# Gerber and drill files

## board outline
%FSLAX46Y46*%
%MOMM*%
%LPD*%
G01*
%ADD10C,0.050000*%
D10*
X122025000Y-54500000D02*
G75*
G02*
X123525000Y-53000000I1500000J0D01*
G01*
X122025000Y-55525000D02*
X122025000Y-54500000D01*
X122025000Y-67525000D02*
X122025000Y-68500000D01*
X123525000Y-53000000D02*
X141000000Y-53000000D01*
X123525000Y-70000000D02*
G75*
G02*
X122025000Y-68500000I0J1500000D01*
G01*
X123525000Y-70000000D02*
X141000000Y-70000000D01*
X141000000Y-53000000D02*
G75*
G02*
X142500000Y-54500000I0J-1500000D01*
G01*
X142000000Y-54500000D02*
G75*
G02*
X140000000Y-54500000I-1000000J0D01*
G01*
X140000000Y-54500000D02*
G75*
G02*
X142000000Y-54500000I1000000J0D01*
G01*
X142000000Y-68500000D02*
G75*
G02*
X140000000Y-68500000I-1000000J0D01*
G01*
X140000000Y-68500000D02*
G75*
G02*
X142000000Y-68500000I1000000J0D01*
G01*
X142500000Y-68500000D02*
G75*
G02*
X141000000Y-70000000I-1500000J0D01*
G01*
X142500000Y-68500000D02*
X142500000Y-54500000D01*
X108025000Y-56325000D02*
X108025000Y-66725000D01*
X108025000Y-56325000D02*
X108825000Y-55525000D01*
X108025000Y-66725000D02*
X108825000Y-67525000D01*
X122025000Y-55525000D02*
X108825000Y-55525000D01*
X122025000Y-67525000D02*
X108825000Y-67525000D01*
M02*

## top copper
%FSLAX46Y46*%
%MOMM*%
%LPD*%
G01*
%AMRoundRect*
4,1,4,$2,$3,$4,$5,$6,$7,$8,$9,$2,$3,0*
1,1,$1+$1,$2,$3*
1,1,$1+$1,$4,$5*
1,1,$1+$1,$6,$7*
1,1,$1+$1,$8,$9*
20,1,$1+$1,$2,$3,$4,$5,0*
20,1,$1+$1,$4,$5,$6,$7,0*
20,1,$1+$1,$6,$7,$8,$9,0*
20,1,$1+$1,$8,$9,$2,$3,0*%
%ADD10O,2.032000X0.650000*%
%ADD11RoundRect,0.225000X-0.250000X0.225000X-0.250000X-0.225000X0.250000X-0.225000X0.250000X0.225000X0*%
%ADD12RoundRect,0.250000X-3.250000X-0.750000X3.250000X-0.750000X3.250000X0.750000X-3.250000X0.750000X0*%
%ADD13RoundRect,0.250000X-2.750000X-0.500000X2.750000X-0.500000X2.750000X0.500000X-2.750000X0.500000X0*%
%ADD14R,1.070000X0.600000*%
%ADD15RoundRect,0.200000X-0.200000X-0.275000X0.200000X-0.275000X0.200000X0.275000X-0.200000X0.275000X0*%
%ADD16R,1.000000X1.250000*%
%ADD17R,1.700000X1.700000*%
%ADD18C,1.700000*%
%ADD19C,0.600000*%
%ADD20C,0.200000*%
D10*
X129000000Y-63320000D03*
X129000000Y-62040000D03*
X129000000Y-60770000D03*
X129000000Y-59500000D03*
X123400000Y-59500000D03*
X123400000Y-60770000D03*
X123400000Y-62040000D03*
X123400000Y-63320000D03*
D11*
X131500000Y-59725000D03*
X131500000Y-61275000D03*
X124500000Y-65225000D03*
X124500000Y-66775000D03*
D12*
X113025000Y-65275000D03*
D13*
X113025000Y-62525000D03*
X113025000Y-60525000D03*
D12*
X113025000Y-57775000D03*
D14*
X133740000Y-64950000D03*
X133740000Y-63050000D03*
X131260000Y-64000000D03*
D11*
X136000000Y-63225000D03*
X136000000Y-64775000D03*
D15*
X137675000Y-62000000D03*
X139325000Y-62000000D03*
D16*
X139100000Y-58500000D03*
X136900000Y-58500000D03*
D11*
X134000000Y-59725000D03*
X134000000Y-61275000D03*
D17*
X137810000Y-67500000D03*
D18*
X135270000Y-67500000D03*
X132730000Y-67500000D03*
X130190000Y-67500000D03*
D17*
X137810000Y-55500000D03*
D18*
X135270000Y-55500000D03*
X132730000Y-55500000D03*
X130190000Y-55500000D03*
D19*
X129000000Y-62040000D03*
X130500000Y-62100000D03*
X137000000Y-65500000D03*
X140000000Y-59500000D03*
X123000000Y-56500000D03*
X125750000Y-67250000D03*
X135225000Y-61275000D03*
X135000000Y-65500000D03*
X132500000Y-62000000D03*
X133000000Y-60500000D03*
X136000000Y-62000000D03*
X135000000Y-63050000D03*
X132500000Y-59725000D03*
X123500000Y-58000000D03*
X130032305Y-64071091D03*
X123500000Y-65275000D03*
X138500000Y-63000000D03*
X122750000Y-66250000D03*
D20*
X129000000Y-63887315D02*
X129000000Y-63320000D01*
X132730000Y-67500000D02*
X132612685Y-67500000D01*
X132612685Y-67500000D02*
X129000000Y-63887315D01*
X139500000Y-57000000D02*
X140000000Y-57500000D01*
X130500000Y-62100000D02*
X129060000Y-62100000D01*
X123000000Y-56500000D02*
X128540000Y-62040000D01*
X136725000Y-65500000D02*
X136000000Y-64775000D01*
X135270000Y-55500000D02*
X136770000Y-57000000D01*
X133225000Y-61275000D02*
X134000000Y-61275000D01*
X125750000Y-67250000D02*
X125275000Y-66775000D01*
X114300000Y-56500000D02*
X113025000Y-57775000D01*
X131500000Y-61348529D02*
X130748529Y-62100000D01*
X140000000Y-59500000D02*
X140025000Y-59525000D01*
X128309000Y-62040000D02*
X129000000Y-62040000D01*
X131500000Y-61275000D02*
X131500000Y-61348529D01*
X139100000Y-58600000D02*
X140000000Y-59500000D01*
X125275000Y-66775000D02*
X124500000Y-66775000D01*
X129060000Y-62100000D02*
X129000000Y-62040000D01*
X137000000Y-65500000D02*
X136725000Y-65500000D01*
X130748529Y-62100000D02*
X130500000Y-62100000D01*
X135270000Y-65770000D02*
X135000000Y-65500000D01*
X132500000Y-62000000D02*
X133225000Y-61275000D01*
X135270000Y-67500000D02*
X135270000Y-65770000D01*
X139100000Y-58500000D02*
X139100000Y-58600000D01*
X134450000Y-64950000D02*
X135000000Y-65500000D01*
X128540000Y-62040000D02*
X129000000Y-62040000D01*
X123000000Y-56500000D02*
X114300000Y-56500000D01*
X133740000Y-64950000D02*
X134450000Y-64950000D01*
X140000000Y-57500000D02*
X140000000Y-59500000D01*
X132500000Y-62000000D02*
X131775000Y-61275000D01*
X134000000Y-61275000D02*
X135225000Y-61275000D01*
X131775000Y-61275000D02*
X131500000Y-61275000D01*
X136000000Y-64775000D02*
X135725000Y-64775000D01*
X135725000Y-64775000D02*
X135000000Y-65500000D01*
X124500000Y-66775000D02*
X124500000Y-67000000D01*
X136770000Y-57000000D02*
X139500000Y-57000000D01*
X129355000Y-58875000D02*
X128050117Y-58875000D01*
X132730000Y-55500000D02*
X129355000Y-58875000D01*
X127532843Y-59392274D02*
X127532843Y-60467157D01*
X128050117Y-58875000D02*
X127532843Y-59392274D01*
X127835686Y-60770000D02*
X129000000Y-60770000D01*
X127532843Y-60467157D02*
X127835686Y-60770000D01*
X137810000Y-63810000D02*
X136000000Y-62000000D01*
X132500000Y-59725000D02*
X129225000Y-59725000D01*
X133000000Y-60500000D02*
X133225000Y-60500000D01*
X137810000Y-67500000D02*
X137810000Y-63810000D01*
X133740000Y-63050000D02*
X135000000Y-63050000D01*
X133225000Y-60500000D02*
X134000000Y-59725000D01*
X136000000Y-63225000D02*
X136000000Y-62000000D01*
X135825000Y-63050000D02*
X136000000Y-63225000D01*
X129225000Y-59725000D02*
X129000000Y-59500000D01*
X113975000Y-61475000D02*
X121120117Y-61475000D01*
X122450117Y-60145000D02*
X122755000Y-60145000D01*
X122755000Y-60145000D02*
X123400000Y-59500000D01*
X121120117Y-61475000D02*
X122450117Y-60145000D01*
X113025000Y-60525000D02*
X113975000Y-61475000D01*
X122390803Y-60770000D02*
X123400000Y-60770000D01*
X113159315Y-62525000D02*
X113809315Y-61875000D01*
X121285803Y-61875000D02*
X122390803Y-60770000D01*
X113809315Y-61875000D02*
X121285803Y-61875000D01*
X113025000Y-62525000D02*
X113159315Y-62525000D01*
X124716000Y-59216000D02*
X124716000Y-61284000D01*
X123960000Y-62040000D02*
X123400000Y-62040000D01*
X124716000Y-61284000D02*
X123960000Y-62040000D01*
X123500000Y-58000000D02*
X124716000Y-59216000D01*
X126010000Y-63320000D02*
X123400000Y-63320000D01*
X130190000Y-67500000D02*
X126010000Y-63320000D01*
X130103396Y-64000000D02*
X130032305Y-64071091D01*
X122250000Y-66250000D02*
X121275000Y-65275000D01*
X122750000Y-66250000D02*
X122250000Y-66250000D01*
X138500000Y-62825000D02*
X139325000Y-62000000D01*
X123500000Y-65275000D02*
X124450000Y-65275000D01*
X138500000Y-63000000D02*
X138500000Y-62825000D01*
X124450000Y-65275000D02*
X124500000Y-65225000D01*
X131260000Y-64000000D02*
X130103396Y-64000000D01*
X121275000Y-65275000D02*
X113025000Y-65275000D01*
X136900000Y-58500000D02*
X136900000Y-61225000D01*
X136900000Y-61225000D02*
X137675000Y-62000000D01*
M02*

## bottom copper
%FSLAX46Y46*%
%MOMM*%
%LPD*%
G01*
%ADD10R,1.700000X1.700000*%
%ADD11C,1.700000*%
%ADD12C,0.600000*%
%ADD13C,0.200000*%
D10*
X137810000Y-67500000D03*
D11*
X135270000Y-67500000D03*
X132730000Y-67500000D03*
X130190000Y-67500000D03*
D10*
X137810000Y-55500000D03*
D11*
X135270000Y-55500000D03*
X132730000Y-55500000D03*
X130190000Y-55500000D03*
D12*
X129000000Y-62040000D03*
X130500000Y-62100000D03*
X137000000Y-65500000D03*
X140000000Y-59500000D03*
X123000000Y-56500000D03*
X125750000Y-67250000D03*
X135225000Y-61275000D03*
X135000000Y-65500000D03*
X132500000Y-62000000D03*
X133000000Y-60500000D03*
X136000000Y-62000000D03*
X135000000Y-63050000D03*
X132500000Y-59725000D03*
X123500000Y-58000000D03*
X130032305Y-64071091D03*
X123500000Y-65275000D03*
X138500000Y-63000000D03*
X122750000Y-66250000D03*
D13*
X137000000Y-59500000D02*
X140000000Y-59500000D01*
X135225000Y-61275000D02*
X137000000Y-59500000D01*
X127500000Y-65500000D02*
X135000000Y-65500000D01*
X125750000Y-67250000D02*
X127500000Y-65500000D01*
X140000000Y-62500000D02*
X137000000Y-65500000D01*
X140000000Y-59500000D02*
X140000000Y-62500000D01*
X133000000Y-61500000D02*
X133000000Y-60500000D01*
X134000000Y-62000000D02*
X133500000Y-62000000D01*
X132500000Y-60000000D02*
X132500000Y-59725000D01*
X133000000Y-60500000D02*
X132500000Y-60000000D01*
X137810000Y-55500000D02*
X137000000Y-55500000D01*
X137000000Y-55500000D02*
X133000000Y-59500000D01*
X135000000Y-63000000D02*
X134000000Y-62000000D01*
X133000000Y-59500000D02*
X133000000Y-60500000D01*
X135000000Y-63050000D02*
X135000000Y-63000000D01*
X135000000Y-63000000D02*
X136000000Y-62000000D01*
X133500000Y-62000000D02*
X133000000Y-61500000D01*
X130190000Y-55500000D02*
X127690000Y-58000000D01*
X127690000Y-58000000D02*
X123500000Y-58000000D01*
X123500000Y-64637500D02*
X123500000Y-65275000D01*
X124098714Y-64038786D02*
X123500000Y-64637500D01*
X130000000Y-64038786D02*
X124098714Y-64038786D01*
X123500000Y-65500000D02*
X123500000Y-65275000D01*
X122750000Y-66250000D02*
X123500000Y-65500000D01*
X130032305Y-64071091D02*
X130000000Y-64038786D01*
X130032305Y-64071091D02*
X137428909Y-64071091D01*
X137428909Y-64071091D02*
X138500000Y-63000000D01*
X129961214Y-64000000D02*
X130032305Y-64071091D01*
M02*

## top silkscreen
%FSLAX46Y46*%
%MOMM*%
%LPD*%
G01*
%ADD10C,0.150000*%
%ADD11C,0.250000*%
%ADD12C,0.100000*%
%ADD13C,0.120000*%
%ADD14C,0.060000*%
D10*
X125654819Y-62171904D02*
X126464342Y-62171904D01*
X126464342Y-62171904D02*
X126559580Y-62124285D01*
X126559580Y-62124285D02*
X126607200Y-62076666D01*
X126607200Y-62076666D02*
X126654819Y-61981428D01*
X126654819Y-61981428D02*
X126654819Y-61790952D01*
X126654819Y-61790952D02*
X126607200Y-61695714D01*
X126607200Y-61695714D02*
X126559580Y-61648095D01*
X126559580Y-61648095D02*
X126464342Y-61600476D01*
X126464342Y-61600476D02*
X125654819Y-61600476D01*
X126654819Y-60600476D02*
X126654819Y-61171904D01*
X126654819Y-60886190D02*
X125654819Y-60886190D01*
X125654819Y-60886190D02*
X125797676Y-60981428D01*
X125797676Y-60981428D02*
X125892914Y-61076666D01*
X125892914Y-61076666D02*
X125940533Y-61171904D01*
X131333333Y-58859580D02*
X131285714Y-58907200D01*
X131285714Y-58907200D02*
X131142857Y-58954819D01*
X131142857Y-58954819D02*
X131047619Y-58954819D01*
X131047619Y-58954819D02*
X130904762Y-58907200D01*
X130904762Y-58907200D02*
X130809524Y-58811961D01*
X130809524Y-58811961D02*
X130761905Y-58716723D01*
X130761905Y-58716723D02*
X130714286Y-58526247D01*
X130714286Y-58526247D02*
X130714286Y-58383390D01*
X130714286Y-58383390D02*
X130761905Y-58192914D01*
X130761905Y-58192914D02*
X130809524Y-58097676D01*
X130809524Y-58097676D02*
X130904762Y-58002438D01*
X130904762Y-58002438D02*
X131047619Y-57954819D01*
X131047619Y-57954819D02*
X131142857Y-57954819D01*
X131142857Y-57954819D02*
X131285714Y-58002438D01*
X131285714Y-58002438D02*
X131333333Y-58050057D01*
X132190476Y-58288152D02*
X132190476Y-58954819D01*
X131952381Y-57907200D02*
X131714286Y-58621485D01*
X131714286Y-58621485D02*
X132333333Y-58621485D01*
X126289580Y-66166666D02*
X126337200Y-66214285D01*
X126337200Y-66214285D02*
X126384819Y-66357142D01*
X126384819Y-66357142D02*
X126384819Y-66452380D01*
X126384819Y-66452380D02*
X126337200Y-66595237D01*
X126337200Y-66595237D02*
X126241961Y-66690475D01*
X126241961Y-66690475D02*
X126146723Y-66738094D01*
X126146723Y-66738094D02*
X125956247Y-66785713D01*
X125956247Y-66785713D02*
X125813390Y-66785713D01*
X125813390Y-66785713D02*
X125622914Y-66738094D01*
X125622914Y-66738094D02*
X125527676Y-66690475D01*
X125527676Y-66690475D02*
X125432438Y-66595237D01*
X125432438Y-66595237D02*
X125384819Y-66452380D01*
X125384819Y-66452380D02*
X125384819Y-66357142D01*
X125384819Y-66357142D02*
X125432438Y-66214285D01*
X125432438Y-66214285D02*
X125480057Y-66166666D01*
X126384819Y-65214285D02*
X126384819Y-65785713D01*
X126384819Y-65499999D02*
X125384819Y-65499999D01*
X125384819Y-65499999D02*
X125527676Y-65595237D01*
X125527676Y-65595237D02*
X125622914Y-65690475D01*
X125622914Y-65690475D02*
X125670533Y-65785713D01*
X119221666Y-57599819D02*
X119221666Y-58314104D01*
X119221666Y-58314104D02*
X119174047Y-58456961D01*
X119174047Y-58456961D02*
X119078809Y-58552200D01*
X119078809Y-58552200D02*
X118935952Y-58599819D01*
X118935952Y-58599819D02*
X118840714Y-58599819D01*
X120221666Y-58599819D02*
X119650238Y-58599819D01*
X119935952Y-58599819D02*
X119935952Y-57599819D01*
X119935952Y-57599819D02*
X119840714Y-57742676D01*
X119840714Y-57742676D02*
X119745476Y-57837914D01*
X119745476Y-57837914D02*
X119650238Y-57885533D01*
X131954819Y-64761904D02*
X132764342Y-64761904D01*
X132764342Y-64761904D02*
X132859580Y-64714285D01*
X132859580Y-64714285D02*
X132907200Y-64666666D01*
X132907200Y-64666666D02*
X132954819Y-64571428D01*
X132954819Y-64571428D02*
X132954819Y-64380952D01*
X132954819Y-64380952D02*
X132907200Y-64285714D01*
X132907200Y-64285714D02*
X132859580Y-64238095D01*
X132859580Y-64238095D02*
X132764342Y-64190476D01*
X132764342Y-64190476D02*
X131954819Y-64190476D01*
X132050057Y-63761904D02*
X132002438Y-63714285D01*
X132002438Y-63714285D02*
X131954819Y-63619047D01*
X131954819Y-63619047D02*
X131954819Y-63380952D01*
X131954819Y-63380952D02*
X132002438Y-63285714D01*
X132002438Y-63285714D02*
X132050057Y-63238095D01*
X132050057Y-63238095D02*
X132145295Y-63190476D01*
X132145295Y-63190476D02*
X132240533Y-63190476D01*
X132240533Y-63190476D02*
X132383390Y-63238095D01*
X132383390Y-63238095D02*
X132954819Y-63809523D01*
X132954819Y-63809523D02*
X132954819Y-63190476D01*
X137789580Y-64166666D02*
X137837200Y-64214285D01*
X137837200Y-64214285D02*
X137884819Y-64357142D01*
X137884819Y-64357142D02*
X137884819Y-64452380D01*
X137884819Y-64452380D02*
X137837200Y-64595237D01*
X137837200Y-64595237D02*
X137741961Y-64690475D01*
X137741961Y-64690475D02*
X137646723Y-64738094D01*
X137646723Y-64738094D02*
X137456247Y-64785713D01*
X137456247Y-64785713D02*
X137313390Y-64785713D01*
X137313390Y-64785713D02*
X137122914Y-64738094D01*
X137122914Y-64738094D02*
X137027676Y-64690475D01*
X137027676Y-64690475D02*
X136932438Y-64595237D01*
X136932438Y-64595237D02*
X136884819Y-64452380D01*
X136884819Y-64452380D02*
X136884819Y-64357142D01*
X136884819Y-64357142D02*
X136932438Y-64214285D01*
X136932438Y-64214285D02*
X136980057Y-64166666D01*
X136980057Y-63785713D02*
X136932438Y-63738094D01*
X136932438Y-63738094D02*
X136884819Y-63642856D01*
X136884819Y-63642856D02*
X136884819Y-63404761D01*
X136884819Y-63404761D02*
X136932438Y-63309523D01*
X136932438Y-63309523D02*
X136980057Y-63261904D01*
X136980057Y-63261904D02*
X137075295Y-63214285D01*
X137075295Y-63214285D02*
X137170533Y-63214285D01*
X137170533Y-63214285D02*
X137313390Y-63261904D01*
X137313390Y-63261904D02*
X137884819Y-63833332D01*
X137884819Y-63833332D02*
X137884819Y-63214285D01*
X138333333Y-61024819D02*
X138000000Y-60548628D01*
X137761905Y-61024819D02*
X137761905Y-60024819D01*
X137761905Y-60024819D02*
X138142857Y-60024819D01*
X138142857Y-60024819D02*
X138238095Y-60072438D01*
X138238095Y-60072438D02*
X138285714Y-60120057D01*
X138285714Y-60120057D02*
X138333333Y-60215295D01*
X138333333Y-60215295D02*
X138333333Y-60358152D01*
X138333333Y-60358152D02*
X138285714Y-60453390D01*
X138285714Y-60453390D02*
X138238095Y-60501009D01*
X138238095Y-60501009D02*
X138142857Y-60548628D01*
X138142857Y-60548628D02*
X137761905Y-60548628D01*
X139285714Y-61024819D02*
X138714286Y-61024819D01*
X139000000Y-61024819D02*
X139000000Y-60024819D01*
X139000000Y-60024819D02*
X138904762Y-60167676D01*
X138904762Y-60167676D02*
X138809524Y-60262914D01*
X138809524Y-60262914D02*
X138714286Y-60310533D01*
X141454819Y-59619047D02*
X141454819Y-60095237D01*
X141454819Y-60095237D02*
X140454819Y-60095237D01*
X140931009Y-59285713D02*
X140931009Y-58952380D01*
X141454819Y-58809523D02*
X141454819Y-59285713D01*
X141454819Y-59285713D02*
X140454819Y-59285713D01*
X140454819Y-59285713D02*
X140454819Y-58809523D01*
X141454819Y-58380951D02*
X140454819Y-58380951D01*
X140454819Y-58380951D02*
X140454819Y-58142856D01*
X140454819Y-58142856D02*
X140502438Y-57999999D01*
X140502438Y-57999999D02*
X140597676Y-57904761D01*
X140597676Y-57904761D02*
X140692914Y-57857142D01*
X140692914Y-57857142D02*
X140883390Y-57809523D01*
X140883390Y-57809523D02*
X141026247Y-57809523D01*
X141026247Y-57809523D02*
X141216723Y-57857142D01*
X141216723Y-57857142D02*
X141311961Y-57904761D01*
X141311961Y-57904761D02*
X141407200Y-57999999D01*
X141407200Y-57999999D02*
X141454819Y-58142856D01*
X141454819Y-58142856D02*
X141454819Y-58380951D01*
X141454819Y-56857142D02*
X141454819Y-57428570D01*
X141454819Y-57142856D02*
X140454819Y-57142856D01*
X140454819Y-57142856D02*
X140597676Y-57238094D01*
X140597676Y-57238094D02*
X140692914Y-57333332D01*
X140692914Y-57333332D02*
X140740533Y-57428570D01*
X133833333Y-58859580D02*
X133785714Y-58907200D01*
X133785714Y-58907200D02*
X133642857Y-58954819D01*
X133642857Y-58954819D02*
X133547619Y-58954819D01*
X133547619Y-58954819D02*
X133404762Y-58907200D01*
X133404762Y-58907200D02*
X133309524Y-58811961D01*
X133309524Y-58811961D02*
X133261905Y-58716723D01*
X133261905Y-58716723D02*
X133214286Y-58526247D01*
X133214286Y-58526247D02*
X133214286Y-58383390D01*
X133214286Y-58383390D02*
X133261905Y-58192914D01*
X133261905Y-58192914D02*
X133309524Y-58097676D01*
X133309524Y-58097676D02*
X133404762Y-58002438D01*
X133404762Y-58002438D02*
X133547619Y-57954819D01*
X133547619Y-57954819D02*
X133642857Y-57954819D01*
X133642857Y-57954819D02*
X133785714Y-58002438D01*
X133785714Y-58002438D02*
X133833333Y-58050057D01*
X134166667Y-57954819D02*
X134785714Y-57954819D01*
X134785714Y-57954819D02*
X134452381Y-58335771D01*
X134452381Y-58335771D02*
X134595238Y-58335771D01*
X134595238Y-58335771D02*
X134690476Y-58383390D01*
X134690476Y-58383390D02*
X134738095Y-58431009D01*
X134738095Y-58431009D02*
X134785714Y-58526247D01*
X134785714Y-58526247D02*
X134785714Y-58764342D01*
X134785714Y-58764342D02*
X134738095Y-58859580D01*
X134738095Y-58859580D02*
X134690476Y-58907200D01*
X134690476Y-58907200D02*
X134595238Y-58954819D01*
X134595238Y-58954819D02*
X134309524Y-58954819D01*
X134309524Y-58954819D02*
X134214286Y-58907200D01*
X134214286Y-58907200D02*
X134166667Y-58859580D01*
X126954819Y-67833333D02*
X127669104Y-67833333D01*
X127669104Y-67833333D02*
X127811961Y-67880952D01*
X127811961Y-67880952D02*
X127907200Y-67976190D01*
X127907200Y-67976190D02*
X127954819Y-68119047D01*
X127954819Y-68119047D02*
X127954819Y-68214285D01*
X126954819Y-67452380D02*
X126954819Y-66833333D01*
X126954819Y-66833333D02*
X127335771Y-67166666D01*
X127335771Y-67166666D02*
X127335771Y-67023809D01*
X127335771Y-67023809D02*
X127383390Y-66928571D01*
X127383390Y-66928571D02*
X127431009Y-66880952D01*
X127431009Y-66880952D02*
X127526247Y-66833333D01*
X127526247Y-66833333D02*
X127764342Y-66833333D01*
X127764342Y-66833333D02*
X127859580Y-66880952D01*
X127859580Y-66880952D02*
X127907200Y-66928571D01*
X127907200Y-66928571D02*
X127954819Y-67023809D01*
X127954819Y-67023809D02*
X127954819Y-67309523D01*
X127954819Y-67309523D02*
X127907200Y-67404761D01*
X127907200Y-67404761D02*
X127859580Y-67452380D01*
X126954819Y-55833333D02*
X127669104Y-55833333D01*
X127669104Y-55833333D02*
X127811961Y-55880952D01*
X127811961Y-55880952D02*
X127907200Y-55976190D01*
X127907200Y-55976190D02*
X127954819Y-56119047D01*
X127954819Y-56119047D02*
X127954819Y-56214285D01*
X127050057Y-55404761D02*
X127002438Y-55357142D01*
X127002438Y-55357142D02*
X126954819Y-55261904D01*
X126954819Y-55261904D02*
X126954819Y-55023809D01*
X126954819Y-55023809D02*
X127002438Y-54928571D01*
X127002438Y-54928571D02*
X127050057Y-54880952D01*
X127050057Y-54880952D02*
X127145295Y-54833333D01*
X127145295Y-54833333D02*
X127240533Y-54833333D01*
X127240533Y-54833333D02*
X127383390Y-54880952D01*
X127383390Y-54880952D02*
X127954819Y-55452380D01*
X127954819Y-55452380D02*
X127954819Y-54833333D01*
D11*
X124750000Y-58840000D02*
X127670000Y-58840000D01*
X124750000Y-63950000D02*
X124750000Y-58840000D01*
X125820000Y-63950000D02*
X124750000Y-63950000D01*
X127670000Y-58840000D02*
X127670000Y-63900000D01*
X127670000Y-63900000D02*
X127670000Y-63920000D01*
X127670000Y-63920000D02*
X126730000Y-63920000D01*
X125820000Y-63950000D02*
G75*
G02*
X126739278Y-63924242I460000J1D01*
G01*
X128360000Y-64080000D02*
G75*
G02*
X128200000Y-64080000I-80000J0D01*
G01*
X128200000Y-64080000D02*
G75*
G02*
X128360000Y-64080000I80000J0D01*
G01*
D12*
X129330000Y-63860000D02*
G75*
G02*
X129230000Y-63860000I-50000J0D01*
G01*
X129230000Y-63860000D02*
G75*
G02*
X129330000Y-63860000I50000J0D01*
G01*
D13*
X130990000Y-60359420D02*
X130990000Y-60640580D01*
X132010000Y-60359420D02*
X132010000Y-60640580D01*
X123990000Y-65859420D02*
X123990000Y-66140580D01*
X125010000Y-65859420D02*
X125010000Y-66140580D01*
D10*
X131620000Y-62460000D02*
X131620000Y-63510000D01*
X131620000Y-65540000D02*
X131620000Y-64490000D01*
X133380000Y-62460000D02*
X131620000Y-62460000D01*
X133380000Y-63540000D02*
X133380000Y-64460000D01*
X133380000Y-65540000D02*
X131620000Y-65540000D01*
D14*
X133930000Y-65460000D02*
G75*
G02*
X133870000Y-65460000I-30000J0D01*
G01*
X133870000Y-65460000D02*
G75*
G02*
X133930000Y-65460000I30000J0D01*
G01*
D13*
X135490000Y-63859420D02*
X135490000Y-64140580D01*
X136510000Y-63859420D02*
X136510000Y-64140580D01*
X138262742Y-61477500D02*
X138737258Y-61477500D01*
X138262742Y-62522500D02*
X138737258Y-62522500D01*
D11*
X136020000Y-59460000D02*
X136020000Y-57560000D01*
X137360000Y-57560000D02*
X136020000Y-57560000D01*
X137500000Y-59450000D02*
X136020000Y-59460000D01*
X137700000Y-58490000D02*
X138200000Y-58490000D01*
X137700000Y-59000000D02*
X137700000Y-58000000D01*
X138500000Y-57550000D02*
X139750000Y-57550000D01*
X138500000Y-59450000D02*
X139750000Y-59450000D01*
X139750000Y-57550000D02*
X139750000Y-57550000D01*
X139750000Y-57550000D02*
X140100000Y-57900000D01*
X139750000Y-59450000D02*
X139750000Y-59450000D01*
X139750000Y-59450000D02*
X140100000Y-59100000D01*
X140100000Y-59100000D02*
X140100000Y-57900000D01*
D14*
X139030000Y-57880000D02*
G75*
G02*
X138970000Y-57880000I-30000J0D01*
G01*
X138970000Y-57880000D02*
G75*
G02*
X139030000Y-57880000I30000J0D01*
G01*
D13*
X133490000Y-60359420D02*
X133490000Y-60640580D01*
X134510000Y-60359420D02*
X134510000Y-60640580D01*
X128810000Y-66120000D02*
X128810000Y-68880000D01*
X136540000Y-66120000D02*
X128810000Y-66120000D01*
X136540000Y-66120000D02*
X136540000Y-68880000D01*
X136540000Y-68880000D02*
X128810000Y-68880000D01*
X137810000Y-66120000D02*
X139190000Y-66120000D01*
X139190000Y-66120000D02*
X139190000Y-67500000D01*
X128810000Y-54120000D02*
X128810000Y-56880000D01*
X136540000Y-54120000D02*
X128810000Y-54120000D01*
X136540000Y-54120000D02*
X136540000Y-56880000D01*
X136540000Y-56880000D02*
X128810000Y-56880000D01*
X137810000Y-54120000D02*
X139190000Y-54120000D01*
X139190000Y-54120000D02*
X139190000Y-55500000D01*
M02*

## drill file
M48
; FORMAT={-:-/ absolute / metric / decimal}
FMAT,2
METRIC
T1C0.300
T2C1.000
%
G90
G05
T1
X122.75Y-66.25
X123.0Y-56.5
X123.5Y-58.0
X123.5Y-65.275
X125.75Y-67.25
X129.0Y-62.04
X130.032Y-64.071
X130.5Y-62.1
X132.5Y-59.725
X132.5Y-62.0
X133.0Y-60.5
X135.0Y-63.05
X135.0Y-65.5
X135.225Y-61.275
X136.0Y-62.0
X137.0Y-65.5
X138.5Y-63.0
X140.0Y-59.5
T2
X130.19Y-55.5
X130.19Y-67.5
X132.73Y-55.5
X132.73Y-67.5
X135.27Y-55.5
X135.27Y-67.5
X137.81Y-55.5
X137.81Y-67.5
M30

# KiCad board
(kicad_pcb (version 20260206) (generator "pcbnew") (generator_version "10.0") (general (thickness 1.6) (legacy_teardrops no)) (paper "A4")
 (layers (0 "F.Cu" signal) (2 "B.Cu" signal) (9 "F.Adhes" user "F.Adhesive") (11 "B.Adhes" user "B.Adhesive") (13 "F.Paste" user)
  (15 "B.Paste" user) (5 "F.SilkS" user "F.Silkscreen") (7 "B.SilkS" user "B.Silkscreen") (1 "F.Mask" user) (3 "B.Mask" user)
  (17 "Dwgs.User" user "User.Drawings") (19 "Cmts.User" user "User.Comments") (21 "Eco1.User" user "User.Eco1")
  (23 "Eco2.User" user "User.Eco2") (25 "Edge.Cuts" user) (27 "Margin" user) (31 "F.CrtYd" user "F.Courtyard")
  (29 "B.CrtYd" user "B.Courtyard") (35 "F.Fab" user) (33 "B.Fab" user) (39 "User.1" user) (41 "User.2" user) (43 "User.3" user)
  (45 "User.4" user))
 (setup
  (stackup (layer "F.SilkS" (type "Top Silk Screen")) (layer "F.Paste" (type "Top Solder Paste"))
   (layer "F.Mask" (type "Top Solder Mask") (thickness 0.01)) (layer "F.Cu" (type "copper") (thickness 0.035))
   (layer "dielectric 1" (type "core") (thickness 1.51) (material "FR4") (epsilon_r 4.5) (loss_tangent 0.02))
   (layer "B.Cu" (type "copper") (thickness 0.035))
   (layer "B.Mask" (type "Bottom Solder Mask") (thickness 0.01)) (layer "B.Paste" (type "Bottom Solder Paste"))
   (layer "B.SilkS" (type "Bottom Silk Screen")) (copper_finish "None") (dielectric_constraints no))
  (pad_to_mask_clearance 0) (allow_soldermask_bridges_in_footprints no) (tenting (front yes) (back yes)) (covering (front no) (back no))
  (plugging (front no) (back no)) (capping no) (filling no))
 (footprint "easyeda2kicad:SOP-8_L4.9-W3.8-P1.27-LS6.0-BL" (layer "F.Cu") (at 126.2 61.41 90)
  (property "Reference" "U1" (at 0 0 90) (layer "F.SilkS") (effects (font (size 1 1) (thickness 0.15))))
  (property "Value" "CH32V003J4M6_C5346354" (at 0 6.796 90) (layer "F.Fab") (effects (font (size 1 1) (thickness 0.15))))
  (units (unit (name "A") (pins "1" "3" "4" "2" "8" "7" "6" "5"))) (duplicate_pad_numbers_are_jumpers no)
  (fp_line (start 2.57 -1.45) (end 2.57 1.47) (stroke (width 0.25) (type solid)) (layer "F.SilkS"))
  (fp_line (start -2.54 -1.45) (end 2.57 -1.45) (stroke (width 0.25) (type solid)) (layer "F.SilkS"))
  (fp_line (start -2.54 -0.38) (end -2.54 -1.45) (stroke (width 0.25) (type solid)) (layer "F.SilkS"))
  (fp_line (start 2.57 1.47) (end -2.49 1.47) (stroke (width 0.25) (type solid)) (layer "F.SilkS"))
  (fp_line (start -2.49 1.47) (end -2.51 1.47) (stroke (width 0.25) (type solid)) (layer "F.SilkS"))
  (fp_line (start -2.51 1.47) (end -2.51 0.53) (stroke (width 0.25) (type solid)) (layer "F.SilkS"))
  (fp_arc (start -2.54 -0.38) (mid -2.08018 0.067116) (end -2.514242 0.539278) (stroke (width 0.25) (type solid)) (layer "F.SilkS"))
  (fp_circle (center -2.67 2.08) (end -2.59 2.08) (stroke (width 0.25) (type solid)) (fill no) (layer "F.SilkS"))
  (fp_circle (center -2.45 3.08) (end -2.4 3.08) (stroke (width 0.1) (type solid)) (fill no) (layer "F.SilkS"))
  (pad "1" smd oval (at -1.91 2.8 90) (size 0.65 2.032) (layers "F.Cu" "F.Mask" "F.Paste") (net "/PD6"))
  (pad "2" smd oval (at -0.63 2.8 90) (size 0.65 2.032) (layers "F.Cu" "F.Mask" "F.Paste") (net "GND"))
  (pad "3" smd oval (at 0.64 2.8 90) (size 0.65 2.032) (layers "F.Cu" "F.Mask" "F.Paste") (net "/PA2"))
  (pad "4" smd oval (at 1.91 2.8 90) (size 0.65 2.032) (layers "F.Cu" "F.Mask" "F.Paste") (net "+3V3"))
  (pad "5" smd oval (at 1.91 -2.8 90) (size 0.65 2.032) (layers "F.Cu" "F.Mask" "F.Paste") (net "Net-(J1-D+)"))
  (pad "6" smd oval (at 0.64 -2.8 90) (size 0.65 2.032) (layers "F.Cu" "F.Mask" "F.Paste") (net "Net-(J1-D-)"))
  (pad "7" smd oval (at -0.63 -2.8 90) (size 0.65 2.032) (layers "F.Cu" "F.Mask" "F.Paste") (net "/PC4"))
  (pad "8" smd oval (at -1.91 -2.8 90) (size 0.65 2.032) (layers "F.Cu" "F.Mask" "F.Paste") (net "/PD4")))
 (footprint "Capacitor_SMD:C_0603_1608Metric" (layer "F.Cu") (at 131.5 60.5 -90)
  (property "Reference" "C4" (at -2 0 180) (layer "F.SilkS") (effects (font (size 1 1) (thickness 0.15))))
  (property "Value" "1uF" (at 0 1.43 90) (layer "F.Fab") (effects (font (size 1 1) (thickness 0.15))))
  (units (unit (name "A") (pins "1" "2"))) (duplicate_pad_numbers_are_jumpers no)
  (fp_line (start -0.14058 0.51) (end 0.14058 0.51) (stroke (width 0.12) (type solid)) (layer "F.SilkS"))
  (fp_line (start -0.14058 -0.51) (end 0.14058 -0.51) (stroke (width 0.12) (type solid)) (layer "F.SilkS"))
  (pad "1" smd roundrect (at -0.775 0 270) (size 0.9 0.95) (layers "F.Cu" "F.Mask" "F.Paste") (roundrect_rratio 0.25) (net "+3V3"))
  (pad "2" smd roundrect (at 0.775 0 270) (size 0.9 0.95) (layers "F.Cu" "F.Mask" "F.Paste") (roundrect_rratio 0.25) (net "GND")))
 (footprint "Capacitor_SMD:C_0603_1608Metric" (layer "F.Cu") (at 124.5 66 -90)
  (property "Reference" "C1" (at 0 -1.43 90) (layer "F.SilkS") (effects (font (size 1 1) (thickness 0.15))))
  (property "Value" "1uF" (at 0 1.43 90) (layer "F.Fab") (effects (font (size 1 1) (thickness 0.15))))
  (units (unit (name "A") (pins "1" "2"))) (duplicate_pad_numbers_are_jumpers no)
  (fp_line (start -0.14058 0.51) (end 0.14058 0.51) (stroke (width 0.12) (type solid)) (layer "F.SilkS"))
  (fp_line (start -0.14058 -0.51) (end 0.14058 -0.51) (stroke (width 0.12) (type solid)) (layer "F.SilkS"))
  (pad "1" smd roundrect (at -0.775 0 270) (size 0.9 0.95) (layers "F.Cu" "F.Mask" "F.Paste") (roundrect_rratio 0.25) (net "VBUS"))
  (pad "2" smd roundrect (at 0.775 0 270) (size 0.9 0.95) (layers "F.Cu" "F.Mask" "F.Paste") (roundrect_rratio 0.25) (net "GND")))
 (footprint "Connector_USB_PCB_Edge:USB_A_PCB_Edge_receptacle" (layer "F.Cu") (at 113.025 61.525)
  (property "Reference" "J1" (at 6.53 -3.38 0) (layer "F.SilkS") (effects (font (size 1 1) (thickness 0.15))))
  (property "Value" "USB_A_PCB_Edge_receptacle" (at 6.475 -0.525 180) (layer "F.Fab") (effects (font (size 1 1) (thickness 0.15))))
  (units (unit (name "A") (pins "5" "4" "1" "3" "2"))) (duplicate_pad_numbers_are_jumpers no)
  (fp_line (start -5 -5.2) (end -5 5.2) (stroke (width 0.05) (type default)) (layer "Edge.Cuts"))
  (fp_line (start -5 -5.2) (end -4.2 -6) (stroke (width 0.05) (type default)) (layer "Edge.Cuts"))
  (fp_line (start -5 5.2) (end -4.2 6) (stroke (width 0.05) (type default)) (layer "Edge.Cuts"))
  (fp_line (start 9 -6) (end -4.2 -6) (stroke (width 0.05) (type default)) (layer "Edge.Cuts"))
  (fp_line (start 9 6) (end -4.2 6) (stroke (width 0.05) (type default)) (layer "Edge.Cuts"))
  (pad "1" smd roundrect (at 0 3.75) (size 7 2) (layers "F.Cu" "F.Mask") (roundrect_rratio 0.125) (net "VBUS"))
  (pad "2" smd roundrect (at 0 1) (size 6 1.5) (layers "F.Cu" "F.Mask") (roundrect_rratio 0.1666666667) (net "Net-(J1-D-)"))
  (pad "3" smd roundrect (at 0 -1) (size 6 1.5) (layers "F.Cu" "F.Mask") (roundrect_rratio 0.1666666667) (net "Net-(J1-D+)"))
  (pad "4" smd roundrect (at 0 -3.75) (size 7 2) (layers "F.Cu" "F.Mask") (roundrect_rratio 0.125) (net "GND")))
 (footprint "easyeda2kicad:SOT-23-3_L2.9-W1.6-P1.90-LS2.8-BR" (layer "F.Cu") (at 132.5 64)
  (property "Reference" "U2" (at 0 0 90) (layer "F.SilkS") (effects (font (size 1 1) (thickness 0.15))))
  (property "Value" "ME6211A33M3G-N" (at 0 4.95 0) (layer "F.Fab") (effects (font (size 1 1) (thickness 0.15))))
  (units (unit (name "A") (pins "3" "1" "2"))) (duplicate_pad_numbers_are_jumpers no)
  (fp_line (start -0.88 -1.54) (end -0.88 -0.49) (stroke (width 0.15) (type solid)) (layer "F.SilkS"))
  (fp_line (start -0.88 1.54) (end -0.88 0.49) (stroke (width 0.15) (type solid)) (layer "F.SilkS"))
  (fp_line (start 0.88 -1.54) (end -0.88 -1.54) (stroke (width 0.15) (type solid)) (layer "F.SilkS"))
  (fp_line (start 0.88 -0.46) (end 0.88 0.46) (stroke (width 0.15) (type solid)) (layer "F.SilkS"))
  (fp_line (start 0.88 1.54) (end -0.88 1.54) (stroke (width 0.15) (type solid)) (layer "F.SilkS"))
  (fp_circle (center 1.4 1.46) (end 1.43 1.46) (stroke (width 0.06) (type solid)) (fill no) (layer "F.SilkS"))
  (pad "1" smd rect (at 1.24 0.95) (size 1.07 0.6) (layers "F.Cu" "F.Mask" "F.Paste") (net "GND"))
  (pad "2" smd rect (at 1.24 -0.95) (size 1.07 0.6) (layers "F.Cu" "F.Mask" "F.Paste") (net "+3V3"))
  (pad "3" smd rect (at -1.24 0) (size 1.07 0.6) (layers "F.Cu" "F.Mask" "F.Paste") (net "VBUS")))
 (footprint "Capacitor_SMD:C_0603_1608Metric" (layer "F.Cu") (at 136 64 -90)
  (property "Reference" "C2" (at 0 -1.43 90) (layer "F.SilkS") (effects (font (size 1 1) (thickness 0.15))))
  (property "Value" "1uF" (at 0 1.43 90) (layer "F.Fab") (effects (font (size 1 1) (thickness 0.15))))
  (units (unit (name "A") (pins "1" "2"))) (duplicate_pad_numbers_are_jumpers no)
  (fp_line (start -0.14058 0.51) (end 0.14058 0.51) (stroke (width 0.12) (type solid)) (layer "F.SilkS"))
  (fp_line (start -0.14058 -0.51) (end 0.14058 -0.51) (stroke (width 0.12) (type solid)) (layer "F.SilkS"))
  (pad "1" smd roundrect (at -0.775 0 270) (size 0.9 0.95) (layers "F.Cu" "F.Mask" "F.Paste") (roundrect_rratio 0.25) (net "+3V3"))
  (pad "2" smd roundrect (at 0.775 0 270) (size 0.9 0.95) (layers "F.Cu" "F.Mask" "F.Paste") (roundrect_rratio 0.25) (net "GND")))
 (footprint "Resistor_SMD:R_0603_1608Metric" (layer "F.Cu") (at 138.5 62)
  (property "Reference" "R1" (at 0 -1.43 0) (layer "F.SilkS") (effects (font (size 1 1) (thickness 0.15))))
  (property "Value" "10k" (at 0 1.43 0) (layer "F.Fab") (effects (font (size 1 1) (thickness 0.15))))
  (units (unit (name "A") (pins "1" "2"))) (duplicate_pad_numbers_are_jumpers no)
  (fp_line (start -0.237258 -0.5225) (end 0.237258 -0.5225) (stroke (width 0.12) (type solid)) (layer "F.SilkS"))
  (fp_line (start -0.237258 0.5225) (end 0.237258 0.5225) (stroke (width 0.12) (type solid)) (layer "F.SilkS"))
  (pad "1" smd roundrect (at -0.825 0) (size 0.8 0.95) (layers "F.Cu" "F.Mask" "F.Paste") (roundrect_rratio 0.25) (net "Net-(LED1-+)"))
  (pad "2" smd roundrect (at 0.825 0) (size 0.8 0.95) (layers "F.Cu" "F.Mask" "F.Paste") (roundrect_rratio 0.25) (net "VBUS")))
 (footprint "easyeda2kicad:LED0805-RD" (layer "F.Cu") (at 138 58.5 180)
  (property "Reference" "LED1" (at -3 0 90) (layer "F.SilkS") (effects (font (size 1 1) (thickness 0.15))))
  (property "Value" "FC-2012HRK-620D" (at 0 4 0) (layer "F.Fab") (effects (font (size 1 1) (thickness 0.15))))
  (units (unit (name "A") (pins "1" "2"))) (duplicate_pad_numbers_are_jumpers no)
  (fp_line (start 1.98 -0.96) (end 1.98 0.94) (stroke (width 0.25) (type solid)) (layer "F.SilkS"))
  (fp_line (start 0.64 0.94) (end 1.98 0.94) (stroke (width 0.25) (type solid)) (layer "F.SilkS"))
  (fp_line (start 0.5 -0.95) (end 1.98 -0.96) (stroke (width 0.25) (type solid)) (layer "F.SilkS"))
  (fp_line (start 0.3 0.01) (end -0.2 0.01) (stroke (width 0.25) (type solid)) (layer "F.SilkS"))
  (fp_line (start 0.3 -0.5) (end 0.3 0.5) (stroke (width 0.25) (type solid)) (layer "F.SilkS"))
  (fp_line (start -0.5 0.95) (end -1.75 0.95) (stroke (width 0.25) (type solid)) (layer "F.SilkS"))
  (fp_line (start -0.5 -0.95) (end -1.75 -0.95) (stroke (width 0.25) (type solid)) (layer "F.SilkS"))
  (fp_line (start -1.75 0.95) (end -1.75 0.95) (stroke (width 0.25) (type solid)) (layer "F.SilkS"))
  (fp_line (start -1.75 0.95) (end -2.1 0.6) (stroke (width 0.25) (type solid)) (layer "F.SilkS"))
  (fp_line (start -1.75 -0.95) (end -1.75 -0.95) (stroke (width 0.25) (type solid)) (layer "F.SilkS"))
  (fp_line (start -1.75 -0.95) (end -2.1 -0.6) (stroke (width 0.25) (type solid)) (layer "F.SilkS"))
  (fp_line (start -2.1 -0.6) (end -2.1 0.6) (stroke (width 0.25) (type solid)) (layer "F.SilkS"))
  (fp_circle (center -1 0.62) (end -0.97 0.62) (stroke (width 0.06) (type solid)) (fill no) (layer "F.SilkS"))
  (pad "1" smd rect (at -1.1 0) (size 1 1.25) (layers "F.Cu" "F.Mask" "F.Paste") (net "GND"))
  (pad "2" smd rect (at 1.1 0) (size 1 1.25) (layers "F.Cu" "F.Mask" "F.Paste") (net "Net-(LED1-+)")))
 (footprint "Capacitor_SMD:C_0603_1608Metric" (layer "F.Cu") (at 134 60.5 -90)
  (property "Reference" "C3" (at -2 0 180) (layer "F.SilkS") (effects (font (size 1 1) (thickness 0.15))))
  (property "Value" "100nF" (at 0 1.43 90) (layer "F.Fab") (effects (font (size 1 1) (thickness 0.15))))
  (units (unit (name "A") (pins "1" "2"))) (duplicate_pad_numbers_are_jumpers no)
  (fp_line (start -0.14058 0.51) (end 0.14058 0.51) (stroke (width 0.12) (type solid)) (layer "F.SilkS"))
  (fp_line (start -0.14058 -0.51) (end 0.14058 -0.51) (stroke (width 0.12) (type solid)) (layer "F.SilkS"))
  (pad "1" smd roundrect (at -0.775 0 270) (size 0.9 0.95) (layers "F.Cu" "F.Mask" "F.Paste") (roundrect_rratio 0.25) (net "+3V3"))
  (pad "2" smd roundrect (at 0.775 0 270) (size 0.9 0.95) (layers "F.Cu" "F.Mask" "F.Paste") (roundrect_rratio 0.25) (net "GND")))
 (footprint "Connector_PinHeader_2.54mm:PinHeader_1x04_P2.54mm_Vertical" (layer "F.Cu") (at 137.81 67.5 -90)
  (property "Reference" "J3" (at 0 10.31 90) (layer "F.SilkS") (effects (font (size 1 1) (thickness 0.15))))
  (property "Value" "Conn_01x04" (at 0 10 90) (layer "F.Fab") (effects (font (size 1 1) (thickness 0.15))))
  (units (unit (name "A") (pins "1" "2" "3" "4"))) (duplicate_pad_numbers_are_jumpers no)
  (fp_line (start -1.38 9) (end 1.38 9) (stroke (width 0.12) (type solid)) (layer "F.SilkS"))
  (fp_line (start -1.38 1.27) (end -1.38 9) (stroke (width 0.12) (type solid)) (layer "F.SilkS"))
  (fp_line (start -1.38 1.27) (end 1.38 1.27) (stroke (width 0.12) (type solid)) (layer "F.SilkS"))
  (fp_line (start 1.38 1.27) (end 1.38 9) (stroke (width 0.12) (type solid)) (layer "F.SilkS"))
  (fp_line (start -1.38 0) (end -1.38 -1.38) (stroke (width 0.12) (type solid)) (layer "F.SilkS"))
  (fp_line (start -1.38 -1.38) (end 0 -1.38) (stroke (width 0.12) (type solid)) (layer "F.SilkS"))
  (pad "1" thru_hole rect (at 0 0 270) (size 1.7 1.7) (drill 1) (layers "*.Cu" "*.Mask") (remove_unused_layers no) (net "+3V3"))
  (pad "2" thru_hole circle (at 0 2.54 270) (size 1.7 1.7) (drill 1) (layers "*.Cu" "*.Mask") (remove_unused_layers no) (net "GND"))
  (pad "3" thru_hole circle (at 0 5.08 270) (size 1.7 1.7) (drill 1) (layers "*.Cu" "*.Mask") (remove_unused_layers no) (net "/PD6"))
  (pad "4" thru_hole circle (at 0 7.62 270) (size 1.7 1.7) (drill 1) (layers "*.Cu" "*.Mask") (remove_unused_layers no) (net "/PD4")))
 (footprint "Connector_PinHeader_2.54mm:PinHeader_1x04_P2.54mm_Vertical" (layer "F.Cu") (at 137.81 55.5 -90)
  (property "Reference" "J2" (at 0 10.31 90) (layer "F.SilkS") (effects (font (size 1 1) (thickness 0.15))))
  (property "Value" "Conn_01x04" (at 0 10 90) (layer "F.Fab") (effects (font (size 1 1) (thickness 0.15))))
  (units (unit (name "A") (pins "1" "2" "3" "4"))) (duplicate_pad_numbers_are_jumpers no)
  (fp_line (start -1.38 9) (end 1.38 9) (stroke (width 0.12) (type solid)) (layer "F.SilkS"))
  (fp_line (start -1.38 1.27) (end -1.38 9) (stroke (width 0.12) (type solid)) (layer "F.SilkS"))
  (fp_line (start -1.38 1.27) (end 1.38 1.27) (stroke (width 0.12) (type solid)) (layer "F.SilkS"))
  (fp_line (start 1.38 1.27) (end 1.38 9) (stroke (width 0.12) (type solid)) (layer "F.SilkS"))
  (fp_line (start -1.38 0) (end -1.38 -1.38) (stroke (width 0.12) (type solid)) (layer "F.SilkS"))
  (fp_line (start -1.38 -1.38) (end 0 -1.38) (stroke (width 0.12) (type solid)) (layer "F.SilkS"))
  (pad "1" thru_hole rect (at 0 0 270) (size 1.7 1.7) (drill 1) (layers "*.Cu" "*.Mask") (remove_unused_layers no) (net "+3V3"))
  (pad "2" thru_hole circle (at 0 2.54 270) (size 1.7 1.7) (drill 1) (layers "*.Cu" "*.Mask") (remove_unused_layers no) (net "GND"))
  (pad "3" thru_hole circle (at 0 5.08 270) (size 1.7 1.7) (drill 1) (layers "*.Cu" "*.Mask") (remove_unused_layers no) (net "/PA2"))
  (pad "4" thru_hole circle (at 0 7.62 270) (size 1.7 1.7) (drill 1) (layers "*.Cu" "*.Mask") (remove_unused_layers no) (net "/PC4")))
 (gr_arc (start 122.025 54.5) (mid 122.46434 53.43934) (end 123.525 53) (stroke (width 0.05) (type default)) (layer "Edge.Cuts"))
 (gr_line (start 122.025 55.525) (end 122.025 54.5) (stroke (width 0.05) (type default)) (layer "Edge.Cuts"))
 (gr_line (start 122.025 67.525) (end 122.025 68.5) (stroke (width 0.05) (type default)) (layer "Edge.Cuts"))
 (gr_line (start 123.525 53) (end 141 53) (stroke (width 0.05) (type default)) (layer "Edge.Cuts"))
 (gr_arc (start 123.525 70) (mid 122.46434 69.56066) (end 122.025 68.5) (stroke (width 0.05) (type default)) (layer "Edge.Cuts"))
 (gr_line (start 123.525 70) (end 141 70) (stroke (width 0.05) (type default)) (layer "Edge.Cuts"))
 (gr_arc (start 141 53) (mid 142.06066 53.43934) (end 142.5 54.5) (stroke (width 0.05) (type default)) (layer "Edge.Cuts"))
 (gr_circle (center 141 54.5) (end 142 54.5) (stroke (width 0.05) (type solid)) (fill no) (layer "Edge.Cuts"))
 (gr_circle (center 141 68.5) (end 142 68.5) (stroke (width 0.05) (type solid)) (fill no) (layer "Edge.Cuts"))
 (gr_arc (start 142.5 68.5) (mid 142.06066 69.56066) (end 141 70) (stroke (width 0.05) (type default)) (layer "Edge.Cuts"))
 (gr_line (start 142.5 68.5) (end 142.5 54.5) (stroke (width 0.05) (type default)) (layer "Edge.Cuts"))
 (segment (start 129 63.887315) (end 129 63.32) (width 0.2) (layer "F.Cu") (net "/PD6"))
 (segment (start 132.73 67.5) (end 132.612685 67.5) (width 0.2) (layer "F.Cu") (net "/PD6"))
 (segment (start 132.612685 67.5) (end 129 63.887315) (width 0.2) (layer "F.Cu") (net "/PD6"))
 (segment (start 139.5 57) (end 140 57.5) (width 0.2) (layer "F.Cu") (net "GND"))
 (segment (start 130.5 62.1) (end 129.06 62.1) (width 0.2) (layer "F.Cu") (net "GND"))
 (segment (start 123 56.5) (end 128.54 62.04) (width 0.2) (layer "F.Cu") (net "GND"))
 (segment (start 136.725 65.5) (end 136 64.775) (width 0.2) (layer "F.Cu") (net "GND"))
 (segment (start 135.27 55.5) (end 136.77 57) (width 0.2) (layer "F.Cu") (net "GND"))
 (segment (start 133.225 61.275) (end 134 61.275) (width 0.2) (layer "F.Cu") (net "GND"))
 (segment (start 125.75 67.25) (end 125.275 66.775) (width 0.2) (layer "F.Cu") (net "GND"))
 (segment (start 114.3 56.5) (end 113.025 57.775) (width 0.2) (layer "F.Cu") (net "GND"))
 (segment (start 131.5 61.348529) (end 130.748529 62.1) (width 0.2) (layer "F.Cu") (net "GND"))
 (segment (start 140 59.5) (end 140.025 59.525) (width 0.2) (layer "F.Cu") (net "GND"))
 (segment (start 128.309 62.04) (end 129 62.04) (width 0.2) (layer "F.Cu") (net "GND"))
 (segment (start 131.5 61.275) (end 131.5 61.348529) (width 0.2) (layer "F.Cu") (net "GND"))
 (segment (start 139.1 58.6) (end 140 59.5) (width 0.2) (layer "F.Cu") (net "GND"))
 (segment (start 125.275 66.775) (end 124.5 66.775) (width 0.2) (layer "F.Cu") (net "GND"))
 (segment (start 129.06 62.1) (end 129 62.04) (width 0.2) (layer "F.Cu") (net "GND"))
 (segment (start 137 65.5) (end 136.725 65.5) (width 0.2) (layer "F.Cu") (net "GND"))
 (segment (start 130.748529 62.1) (end 130.5 62.1) (width 0.2) (layer "F.Cu") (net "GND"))
 (segment (start 135.27 65.77) (end 135 65.5) (width 0.2) (layer "F.Cu") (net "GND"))
 (segment (start 132.5 62) (end 133.225 61.275) (width 0.2) (layer "F.Cu") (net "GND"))
 (segment (start 135.27 67.5) (end 135.27 65.77) (width 0.2) (layer "F.Cu") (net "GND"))
 (segment (start 139.1 58.5) (end 139.1 58.6) (width 0.2) (layer "F.Cu") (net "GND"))
 (segment (start 134.45 64.95) (end 135 65.5) (width 0.2) (layer "F.Cu") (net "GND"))
 (segment (start 128.54 62.04) (end 129 62.04) (width 0.2) (layer "F.Cu") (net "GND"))
 (segment (start 123 56.5) (end 114.3 56.5) (width 0.2) (layer "F.Cu") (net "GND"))
 (segment (start 133.74 64.95) (end 134.45 64.95) (width 0.2) (layer "F.Cu") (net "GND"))
 (segment (start 140 57.5) (end 140 59.5) (width 0.2) (layer "F.Cu") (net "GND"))
 (segment (start 132.5 62) (end 131.775 61.275) (width 0.2) (layer "F.Cu") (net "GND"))
 (segment (start 134 61.275) (end 135.225 61.275) (width 0.2) (layer "F.Cu") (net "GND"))
 (segment (start 131.775 61.275) (end 131.5 61.275) (width 0.2) (layer "F.Cu") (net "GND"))
 (segment (start 136 64.775) (end 135.725 64.775) (width 0.2) (layer "F.Cu") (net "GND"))
 (segment (start 135.725 64.775) (end 135 65.5) (width 0.2) (layer "F.Cu") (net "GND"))
 (segment (start 124.5 66.775) (end 124.5 67) (width 0.2) (layer "F.Cu") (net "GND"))
 (segment (start 136.77 57) (end 139.5 57) (width 0.2) (layer "F.Cu") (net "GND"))
 (via (at 129 62.04) (size 0.6) (drill 0.3) (layers "F.Cu" "B.Cu") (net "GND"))
 (via (at 130.5 62.1) (size 0.6) (drill 0.3) (layers "F.Cu" "B.Cu") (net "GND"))
 (via (at 137 65.5) (size 0.6) (drill 0.3) (layers "F.Cu" "B.Cu") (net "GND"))
 (via (at 140 59.5) (size 0.6) (drill 0.3) (layers "F.Cu" "B.Cu") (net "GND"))
 (via (at 123 56.5) (size 0.6) (drill 0.3) (layers "F.Cu" "B.Cu") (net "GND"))
 (via (at 125.75 67.25) (size 0.6) (drill 0.3) (layers "F.Cu" "B.Cu") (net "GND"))
 (via (at 135.225 61.275) (size 0.6) (drill 0.3) (layers "F.Cu" "B.Cu") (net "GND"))
 (via (at 135 65.5) (size 0.6) (drill 0.3) (layers "F.Cu" "B.Cu") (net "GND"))
 (via (at 132.5 62) (size 0.6) (drill 0.3) (layers "F.Cu" "B.Cu") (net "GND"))
 (segment (start 137 59.5) (end 140 59.5) (width 0.2) (layer "B.Cu") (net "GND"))
 (segment (start 135.225 61.275) (end 137 59.5) (width 0.2) (layer "B.Cu") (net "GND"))
 (segment (start 127.5 65.5) (end 135 65.5) (width 0.2) (layer "B.Cu") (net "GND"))
 (segment (start 125.75 67.25) (end 127.5 65.5) (width 0.2) (layer "B.Cu") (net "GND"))
 (segment (start 140 62.5) (end 137 65.5) (width 0.2) (layer "B.Cu") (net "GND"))
 (segment (start 140 59.5) (end 140 62.5) (width 0.2) (layer "B.Cu") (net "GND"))
 (segment (start 129.355 58.875) (end 128.050117 58.875) (width 0.2) (layer "F.Cu") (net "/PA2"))
 (segment (start 132.73 55.5) (end 129.355 58.875) (width 0.2) (layer "F.Cu") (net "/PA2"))
 (segment (start 127.532843 59.392274) (end 127.532843 60.467157) (width 0.2) (layer "F.Cu") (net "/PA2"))
 (segment (start 128.050117 58.875) (end 127.532843 59.392274) (width 0.2) (layer "F.Cu") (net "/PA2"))
 (segment (start 127.835686 60.77) (end 129 60.77) (width 0.2) (layer "F.Cu") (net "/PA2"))
 (segment (start 127.532843 60.467157) (end 127.835686 60.77) (width 0.2) (layer "F.Cu") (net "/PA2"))
 (segment (start 137.81 63.81) (end 136 62) (width 0.2) (layer "F.Cu") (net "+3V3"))
 (segment (start 132.5 59.725) (end 129.225 59.725) (width 0.2) (layer "F.Cu") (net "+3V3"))
 (segment (start 133 60.5) (end 133.225 60.5) (width 0.2) (layer "F.Cu") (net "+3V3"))
 (segment (start 137.81 67.5) (end 137.81 63.81) (width 0.2) (layer "F.Cu") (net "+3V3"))
 (segment (start 133.74 63.05) (end 135 63.05) (width 0.2) (layer "F.Cu") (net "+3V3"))
 (segment (start 133.225 60.5) (end 134 59.725) (width 0.2) (layer "F.Cu") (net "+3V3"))
 (segment (start 136 63.225) (end 136 62) (width 0.2) (layer "F.Cu") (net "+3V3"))
 (segment (start 135.825 63.05) (end 136 63.225) (width 0.2) (layer "F.Cu") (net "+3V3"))
 (segment (start 129.225 59.725) (end 129 59.5) (width 0.2) (layer "F.Cu") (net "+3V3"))
 (via (at 133 60.5) (size 0.6) (drill 0.3) (layers "F.Cu" "B.Cu") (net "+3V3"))
 (via (at 136 62) (size 0.6) (drill 0.3) (layers "F.Cu" "B.Cu") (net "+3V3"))
 (via (at 135 63.05) (size 0.6) (drill 0.3) (layers "F.Cu" "B.Cu") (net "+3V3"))
 (via (at 132.5 59.725) (size 0.6) (drill 0.3) (layers "F.Cu" "B.Cu") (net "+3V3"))
 (segment (start 133 61.5) (end 133 60.5) (width 0.2) (layer "B.Cu") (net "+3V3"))
 (segment (start 134 62) (end 133.5 62) (width 0.2) (layer "B.Cu") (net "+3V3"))
 (segment (start 132.5 60) (end 132.5 59.725) (width 0.2) (layer "B.Cu") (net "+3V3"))
 (segment (start 133 60.5) (end 132.5 60) (width 0.2) (layer "B.Cu") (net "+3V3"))
 (segment (start 137.81 55.5) (end 137 55.5) (width 0.2) (layer "B.Cu") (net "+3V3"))
 (segment (start 137 55.5) (end 133 59.5) (width 0.2) (layer "B.Cu") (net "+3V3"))
 (segment (start 135 63) (end 134 62) (width 0.2) (layer "B.Cu") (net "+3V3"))
 (segment (start 133 59.5) (end 133 60.5) (width 0.2) (layer "B.Cu") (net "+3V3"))
 (segment (start 135 63.05) (end 135 63) (width 0.2) (layer "B.Cu") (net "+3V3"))
 (segment (start 135 63) (end 136 62) (width 0.2) (layer "B.Cu") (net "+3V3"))
 (segment (start 133.5 62) (end 133 61.5) (width 0.2) (layer "B.Cu") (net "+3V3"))
 (segment (start 113.975 61.475) (end 121.120117 61.475) (width 0.2) (layer "F.Cu") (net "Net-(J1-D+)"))
 (segment (start 122.450117 60.145) (end 122.755 60.145) (width 0.2) (layer "F.Cu") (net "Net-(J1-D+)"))
 (segment (start 122.755 60.145) (end 123.4 59.5) (width 0.2) (layer "F.Cu") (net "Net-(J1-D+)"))
 (segment (start 121.120117 61.475) (end 122.450117 60.145) (width 0.2) (layer "F.Cu") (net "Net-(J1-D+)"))
 (segment (start 113.025 60.525) (end 113.975 61.475) (width 0.2) (layer "F.Cu") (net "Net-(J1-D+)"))
 (segment (start 122.390803 60.77) (end 123.4 60.77) (width 0.2) (layer "F.Cu") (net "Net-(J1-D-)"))
 (segment (start 113.159315 62.525) (end 113.809315 61.875) (width 0.2) (layer "F.Cu") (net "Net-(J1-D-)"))
 (segment (start 121.285803 61.875) (end 122.390803 60.77) (width 0.2) (layer "F.Cu") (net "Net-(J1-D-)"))
 (segment (start 113.809315 61.875) (end 121.285803 61.875) (width 0.2) (layer "F.Cu") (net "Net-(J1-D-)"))
 (segment (start 113.025 62.525) (end 113.159315 62.525) (width 0.2) (layer "F.Cu") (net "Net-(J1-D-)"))
 (segment (start 124.716 59.216) (end 124.716 61.284) (width 0.2) (layer "F.Cu") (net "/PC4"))
 (segment (start 123.96 62.04) (end 123.4 62.04) (width 0.2) (layer "F.Cu") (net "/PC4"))
 (segment (start 124.716 61.284) (end 123.96 62.04) (width 0.2) (layer "F.Cu") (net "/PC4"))
 (segment (start 123.5 58) (end 124.716 59.216) (width 0.2) (layer "F.Cu") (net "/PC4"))
 (via (at 123.5 58) (size 0.6) (drill 0.3) (layers "F.Cu" "B.Cu") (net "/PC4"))
 (segment (start 130.19 55.5) (end 127.69 58) (width 0.2) (layer "B.Cu") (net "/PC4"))
 (segment (start 127.69 58) (end 123.5 58) (width 0.2) (layer "B.Cu") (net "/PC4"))
 (segment (start 126.01 63.32) (end 123.4 63.32) (width 0.2) (layer "F.Cu") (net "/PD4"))
 (segment (start 130.19 67.5) (end 126.01 63.32) (width 0.2) (layer "F.Cu") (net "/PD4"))
 (segment (start 130.103396 64) (end 130.032305 64.071091) (width 0.2) (layer "F.Cu") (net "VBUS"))
 (segment (start 122.25 66.25) (end 121.275 65.275) (width 0.2) (layer "F.Cu") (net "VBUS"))
 (segment (start 122.75 66.25) (end 122.25 66.25) (width 0.2) (layer "F.Cu") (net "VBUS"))
 (segment (start 138.5 62.825) (end 139.325 62) (width 0.2) (layer "F.Cu") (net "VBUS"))
 (segment (start 123.5 65.275) (end 124.45 65.275) (width 0.2) (layer "F.Cu") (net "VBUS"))
 (segment (start 138.5 63) (end 138.5 62.825) (width 0.2) (layer "F.Cu") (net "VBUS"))
 (segment (start 124.45 65.275) (end 124.5 65.225) (width 0.2) (layer "F.Cu") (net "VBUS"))
 (segment (start 131.26 64) (end 130.103396 64) (width 0.2) (layer "F.Cu") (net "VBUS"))
 (segment (start 121.275 65.275) (end 113.025 65.275) (width 0.2) (layer "F.Cu") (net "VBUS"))
 (via (at 130.032305 64.071091) (size 0.6) (drill 0.3) (layers "F.Cu" "B.Cu") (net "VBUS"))
 (via (at 123.5 65.275) (size 0.6) (drill 0.3) (layers "F.Cu" "B.Cu") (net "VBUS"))
 (via (at 138.5 63) (size 0.6) (drill 0.3) (layers "F.Cu" "B.Cu") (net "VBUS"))
 (via (at 122.75 66.25) (size 0.6) (drill 0.3) (layers "F.Cu" "B.Cu") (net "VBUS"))
 (segment (start 123.5 64.6375) (end 123.5 65.275) (width 0.2) (layer "B.Cu") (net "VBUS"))
 (segment (start 124.098714 64.038786) (end 123.5 64.6375) (width 0.2) (layer "B.Cu") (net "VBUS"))
 (segment (start 130 64.038786) (end 124.098714 64.038786) (width 0.2) (layer "B.Cu") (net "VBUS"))
 (segment (start 123.5 65.5) (end 123.5 65.275) (width 0.2) (layer "B.Cu") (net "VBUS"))
 (segment (start 122.75 66.25) (end 123.5 65.5) (width 0.2) (layer "B.Cu") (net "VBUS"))
 (segment (start 130.032305 64.071091) (end 130 64.038786) (width 0.2) (layer "B.Cu") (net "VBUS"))
 (segment (start 130.032305 64.071091) (end 137.428909 64.071091) (width 0.2) (layer "B.Cu") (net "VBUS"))
 (segment (start 137.428909 64.071091) (end 138.5 63) (width 0.2) (layer "B.Cu") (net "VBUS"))
 (segment (start 129.961214 64) (end 130.032305 64.071091) (width 0.2) (layer "B.Cu") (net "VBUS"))
 (segment (start 136.9 58.5) (end 136.9 61.225) (width 0.2) (layer "F.Cu") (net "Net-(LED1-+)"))
 (segment (start 136.9 61.225) (end 137.675 62) (width 0.2) (layer "F.Cu") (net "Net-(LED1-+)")))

